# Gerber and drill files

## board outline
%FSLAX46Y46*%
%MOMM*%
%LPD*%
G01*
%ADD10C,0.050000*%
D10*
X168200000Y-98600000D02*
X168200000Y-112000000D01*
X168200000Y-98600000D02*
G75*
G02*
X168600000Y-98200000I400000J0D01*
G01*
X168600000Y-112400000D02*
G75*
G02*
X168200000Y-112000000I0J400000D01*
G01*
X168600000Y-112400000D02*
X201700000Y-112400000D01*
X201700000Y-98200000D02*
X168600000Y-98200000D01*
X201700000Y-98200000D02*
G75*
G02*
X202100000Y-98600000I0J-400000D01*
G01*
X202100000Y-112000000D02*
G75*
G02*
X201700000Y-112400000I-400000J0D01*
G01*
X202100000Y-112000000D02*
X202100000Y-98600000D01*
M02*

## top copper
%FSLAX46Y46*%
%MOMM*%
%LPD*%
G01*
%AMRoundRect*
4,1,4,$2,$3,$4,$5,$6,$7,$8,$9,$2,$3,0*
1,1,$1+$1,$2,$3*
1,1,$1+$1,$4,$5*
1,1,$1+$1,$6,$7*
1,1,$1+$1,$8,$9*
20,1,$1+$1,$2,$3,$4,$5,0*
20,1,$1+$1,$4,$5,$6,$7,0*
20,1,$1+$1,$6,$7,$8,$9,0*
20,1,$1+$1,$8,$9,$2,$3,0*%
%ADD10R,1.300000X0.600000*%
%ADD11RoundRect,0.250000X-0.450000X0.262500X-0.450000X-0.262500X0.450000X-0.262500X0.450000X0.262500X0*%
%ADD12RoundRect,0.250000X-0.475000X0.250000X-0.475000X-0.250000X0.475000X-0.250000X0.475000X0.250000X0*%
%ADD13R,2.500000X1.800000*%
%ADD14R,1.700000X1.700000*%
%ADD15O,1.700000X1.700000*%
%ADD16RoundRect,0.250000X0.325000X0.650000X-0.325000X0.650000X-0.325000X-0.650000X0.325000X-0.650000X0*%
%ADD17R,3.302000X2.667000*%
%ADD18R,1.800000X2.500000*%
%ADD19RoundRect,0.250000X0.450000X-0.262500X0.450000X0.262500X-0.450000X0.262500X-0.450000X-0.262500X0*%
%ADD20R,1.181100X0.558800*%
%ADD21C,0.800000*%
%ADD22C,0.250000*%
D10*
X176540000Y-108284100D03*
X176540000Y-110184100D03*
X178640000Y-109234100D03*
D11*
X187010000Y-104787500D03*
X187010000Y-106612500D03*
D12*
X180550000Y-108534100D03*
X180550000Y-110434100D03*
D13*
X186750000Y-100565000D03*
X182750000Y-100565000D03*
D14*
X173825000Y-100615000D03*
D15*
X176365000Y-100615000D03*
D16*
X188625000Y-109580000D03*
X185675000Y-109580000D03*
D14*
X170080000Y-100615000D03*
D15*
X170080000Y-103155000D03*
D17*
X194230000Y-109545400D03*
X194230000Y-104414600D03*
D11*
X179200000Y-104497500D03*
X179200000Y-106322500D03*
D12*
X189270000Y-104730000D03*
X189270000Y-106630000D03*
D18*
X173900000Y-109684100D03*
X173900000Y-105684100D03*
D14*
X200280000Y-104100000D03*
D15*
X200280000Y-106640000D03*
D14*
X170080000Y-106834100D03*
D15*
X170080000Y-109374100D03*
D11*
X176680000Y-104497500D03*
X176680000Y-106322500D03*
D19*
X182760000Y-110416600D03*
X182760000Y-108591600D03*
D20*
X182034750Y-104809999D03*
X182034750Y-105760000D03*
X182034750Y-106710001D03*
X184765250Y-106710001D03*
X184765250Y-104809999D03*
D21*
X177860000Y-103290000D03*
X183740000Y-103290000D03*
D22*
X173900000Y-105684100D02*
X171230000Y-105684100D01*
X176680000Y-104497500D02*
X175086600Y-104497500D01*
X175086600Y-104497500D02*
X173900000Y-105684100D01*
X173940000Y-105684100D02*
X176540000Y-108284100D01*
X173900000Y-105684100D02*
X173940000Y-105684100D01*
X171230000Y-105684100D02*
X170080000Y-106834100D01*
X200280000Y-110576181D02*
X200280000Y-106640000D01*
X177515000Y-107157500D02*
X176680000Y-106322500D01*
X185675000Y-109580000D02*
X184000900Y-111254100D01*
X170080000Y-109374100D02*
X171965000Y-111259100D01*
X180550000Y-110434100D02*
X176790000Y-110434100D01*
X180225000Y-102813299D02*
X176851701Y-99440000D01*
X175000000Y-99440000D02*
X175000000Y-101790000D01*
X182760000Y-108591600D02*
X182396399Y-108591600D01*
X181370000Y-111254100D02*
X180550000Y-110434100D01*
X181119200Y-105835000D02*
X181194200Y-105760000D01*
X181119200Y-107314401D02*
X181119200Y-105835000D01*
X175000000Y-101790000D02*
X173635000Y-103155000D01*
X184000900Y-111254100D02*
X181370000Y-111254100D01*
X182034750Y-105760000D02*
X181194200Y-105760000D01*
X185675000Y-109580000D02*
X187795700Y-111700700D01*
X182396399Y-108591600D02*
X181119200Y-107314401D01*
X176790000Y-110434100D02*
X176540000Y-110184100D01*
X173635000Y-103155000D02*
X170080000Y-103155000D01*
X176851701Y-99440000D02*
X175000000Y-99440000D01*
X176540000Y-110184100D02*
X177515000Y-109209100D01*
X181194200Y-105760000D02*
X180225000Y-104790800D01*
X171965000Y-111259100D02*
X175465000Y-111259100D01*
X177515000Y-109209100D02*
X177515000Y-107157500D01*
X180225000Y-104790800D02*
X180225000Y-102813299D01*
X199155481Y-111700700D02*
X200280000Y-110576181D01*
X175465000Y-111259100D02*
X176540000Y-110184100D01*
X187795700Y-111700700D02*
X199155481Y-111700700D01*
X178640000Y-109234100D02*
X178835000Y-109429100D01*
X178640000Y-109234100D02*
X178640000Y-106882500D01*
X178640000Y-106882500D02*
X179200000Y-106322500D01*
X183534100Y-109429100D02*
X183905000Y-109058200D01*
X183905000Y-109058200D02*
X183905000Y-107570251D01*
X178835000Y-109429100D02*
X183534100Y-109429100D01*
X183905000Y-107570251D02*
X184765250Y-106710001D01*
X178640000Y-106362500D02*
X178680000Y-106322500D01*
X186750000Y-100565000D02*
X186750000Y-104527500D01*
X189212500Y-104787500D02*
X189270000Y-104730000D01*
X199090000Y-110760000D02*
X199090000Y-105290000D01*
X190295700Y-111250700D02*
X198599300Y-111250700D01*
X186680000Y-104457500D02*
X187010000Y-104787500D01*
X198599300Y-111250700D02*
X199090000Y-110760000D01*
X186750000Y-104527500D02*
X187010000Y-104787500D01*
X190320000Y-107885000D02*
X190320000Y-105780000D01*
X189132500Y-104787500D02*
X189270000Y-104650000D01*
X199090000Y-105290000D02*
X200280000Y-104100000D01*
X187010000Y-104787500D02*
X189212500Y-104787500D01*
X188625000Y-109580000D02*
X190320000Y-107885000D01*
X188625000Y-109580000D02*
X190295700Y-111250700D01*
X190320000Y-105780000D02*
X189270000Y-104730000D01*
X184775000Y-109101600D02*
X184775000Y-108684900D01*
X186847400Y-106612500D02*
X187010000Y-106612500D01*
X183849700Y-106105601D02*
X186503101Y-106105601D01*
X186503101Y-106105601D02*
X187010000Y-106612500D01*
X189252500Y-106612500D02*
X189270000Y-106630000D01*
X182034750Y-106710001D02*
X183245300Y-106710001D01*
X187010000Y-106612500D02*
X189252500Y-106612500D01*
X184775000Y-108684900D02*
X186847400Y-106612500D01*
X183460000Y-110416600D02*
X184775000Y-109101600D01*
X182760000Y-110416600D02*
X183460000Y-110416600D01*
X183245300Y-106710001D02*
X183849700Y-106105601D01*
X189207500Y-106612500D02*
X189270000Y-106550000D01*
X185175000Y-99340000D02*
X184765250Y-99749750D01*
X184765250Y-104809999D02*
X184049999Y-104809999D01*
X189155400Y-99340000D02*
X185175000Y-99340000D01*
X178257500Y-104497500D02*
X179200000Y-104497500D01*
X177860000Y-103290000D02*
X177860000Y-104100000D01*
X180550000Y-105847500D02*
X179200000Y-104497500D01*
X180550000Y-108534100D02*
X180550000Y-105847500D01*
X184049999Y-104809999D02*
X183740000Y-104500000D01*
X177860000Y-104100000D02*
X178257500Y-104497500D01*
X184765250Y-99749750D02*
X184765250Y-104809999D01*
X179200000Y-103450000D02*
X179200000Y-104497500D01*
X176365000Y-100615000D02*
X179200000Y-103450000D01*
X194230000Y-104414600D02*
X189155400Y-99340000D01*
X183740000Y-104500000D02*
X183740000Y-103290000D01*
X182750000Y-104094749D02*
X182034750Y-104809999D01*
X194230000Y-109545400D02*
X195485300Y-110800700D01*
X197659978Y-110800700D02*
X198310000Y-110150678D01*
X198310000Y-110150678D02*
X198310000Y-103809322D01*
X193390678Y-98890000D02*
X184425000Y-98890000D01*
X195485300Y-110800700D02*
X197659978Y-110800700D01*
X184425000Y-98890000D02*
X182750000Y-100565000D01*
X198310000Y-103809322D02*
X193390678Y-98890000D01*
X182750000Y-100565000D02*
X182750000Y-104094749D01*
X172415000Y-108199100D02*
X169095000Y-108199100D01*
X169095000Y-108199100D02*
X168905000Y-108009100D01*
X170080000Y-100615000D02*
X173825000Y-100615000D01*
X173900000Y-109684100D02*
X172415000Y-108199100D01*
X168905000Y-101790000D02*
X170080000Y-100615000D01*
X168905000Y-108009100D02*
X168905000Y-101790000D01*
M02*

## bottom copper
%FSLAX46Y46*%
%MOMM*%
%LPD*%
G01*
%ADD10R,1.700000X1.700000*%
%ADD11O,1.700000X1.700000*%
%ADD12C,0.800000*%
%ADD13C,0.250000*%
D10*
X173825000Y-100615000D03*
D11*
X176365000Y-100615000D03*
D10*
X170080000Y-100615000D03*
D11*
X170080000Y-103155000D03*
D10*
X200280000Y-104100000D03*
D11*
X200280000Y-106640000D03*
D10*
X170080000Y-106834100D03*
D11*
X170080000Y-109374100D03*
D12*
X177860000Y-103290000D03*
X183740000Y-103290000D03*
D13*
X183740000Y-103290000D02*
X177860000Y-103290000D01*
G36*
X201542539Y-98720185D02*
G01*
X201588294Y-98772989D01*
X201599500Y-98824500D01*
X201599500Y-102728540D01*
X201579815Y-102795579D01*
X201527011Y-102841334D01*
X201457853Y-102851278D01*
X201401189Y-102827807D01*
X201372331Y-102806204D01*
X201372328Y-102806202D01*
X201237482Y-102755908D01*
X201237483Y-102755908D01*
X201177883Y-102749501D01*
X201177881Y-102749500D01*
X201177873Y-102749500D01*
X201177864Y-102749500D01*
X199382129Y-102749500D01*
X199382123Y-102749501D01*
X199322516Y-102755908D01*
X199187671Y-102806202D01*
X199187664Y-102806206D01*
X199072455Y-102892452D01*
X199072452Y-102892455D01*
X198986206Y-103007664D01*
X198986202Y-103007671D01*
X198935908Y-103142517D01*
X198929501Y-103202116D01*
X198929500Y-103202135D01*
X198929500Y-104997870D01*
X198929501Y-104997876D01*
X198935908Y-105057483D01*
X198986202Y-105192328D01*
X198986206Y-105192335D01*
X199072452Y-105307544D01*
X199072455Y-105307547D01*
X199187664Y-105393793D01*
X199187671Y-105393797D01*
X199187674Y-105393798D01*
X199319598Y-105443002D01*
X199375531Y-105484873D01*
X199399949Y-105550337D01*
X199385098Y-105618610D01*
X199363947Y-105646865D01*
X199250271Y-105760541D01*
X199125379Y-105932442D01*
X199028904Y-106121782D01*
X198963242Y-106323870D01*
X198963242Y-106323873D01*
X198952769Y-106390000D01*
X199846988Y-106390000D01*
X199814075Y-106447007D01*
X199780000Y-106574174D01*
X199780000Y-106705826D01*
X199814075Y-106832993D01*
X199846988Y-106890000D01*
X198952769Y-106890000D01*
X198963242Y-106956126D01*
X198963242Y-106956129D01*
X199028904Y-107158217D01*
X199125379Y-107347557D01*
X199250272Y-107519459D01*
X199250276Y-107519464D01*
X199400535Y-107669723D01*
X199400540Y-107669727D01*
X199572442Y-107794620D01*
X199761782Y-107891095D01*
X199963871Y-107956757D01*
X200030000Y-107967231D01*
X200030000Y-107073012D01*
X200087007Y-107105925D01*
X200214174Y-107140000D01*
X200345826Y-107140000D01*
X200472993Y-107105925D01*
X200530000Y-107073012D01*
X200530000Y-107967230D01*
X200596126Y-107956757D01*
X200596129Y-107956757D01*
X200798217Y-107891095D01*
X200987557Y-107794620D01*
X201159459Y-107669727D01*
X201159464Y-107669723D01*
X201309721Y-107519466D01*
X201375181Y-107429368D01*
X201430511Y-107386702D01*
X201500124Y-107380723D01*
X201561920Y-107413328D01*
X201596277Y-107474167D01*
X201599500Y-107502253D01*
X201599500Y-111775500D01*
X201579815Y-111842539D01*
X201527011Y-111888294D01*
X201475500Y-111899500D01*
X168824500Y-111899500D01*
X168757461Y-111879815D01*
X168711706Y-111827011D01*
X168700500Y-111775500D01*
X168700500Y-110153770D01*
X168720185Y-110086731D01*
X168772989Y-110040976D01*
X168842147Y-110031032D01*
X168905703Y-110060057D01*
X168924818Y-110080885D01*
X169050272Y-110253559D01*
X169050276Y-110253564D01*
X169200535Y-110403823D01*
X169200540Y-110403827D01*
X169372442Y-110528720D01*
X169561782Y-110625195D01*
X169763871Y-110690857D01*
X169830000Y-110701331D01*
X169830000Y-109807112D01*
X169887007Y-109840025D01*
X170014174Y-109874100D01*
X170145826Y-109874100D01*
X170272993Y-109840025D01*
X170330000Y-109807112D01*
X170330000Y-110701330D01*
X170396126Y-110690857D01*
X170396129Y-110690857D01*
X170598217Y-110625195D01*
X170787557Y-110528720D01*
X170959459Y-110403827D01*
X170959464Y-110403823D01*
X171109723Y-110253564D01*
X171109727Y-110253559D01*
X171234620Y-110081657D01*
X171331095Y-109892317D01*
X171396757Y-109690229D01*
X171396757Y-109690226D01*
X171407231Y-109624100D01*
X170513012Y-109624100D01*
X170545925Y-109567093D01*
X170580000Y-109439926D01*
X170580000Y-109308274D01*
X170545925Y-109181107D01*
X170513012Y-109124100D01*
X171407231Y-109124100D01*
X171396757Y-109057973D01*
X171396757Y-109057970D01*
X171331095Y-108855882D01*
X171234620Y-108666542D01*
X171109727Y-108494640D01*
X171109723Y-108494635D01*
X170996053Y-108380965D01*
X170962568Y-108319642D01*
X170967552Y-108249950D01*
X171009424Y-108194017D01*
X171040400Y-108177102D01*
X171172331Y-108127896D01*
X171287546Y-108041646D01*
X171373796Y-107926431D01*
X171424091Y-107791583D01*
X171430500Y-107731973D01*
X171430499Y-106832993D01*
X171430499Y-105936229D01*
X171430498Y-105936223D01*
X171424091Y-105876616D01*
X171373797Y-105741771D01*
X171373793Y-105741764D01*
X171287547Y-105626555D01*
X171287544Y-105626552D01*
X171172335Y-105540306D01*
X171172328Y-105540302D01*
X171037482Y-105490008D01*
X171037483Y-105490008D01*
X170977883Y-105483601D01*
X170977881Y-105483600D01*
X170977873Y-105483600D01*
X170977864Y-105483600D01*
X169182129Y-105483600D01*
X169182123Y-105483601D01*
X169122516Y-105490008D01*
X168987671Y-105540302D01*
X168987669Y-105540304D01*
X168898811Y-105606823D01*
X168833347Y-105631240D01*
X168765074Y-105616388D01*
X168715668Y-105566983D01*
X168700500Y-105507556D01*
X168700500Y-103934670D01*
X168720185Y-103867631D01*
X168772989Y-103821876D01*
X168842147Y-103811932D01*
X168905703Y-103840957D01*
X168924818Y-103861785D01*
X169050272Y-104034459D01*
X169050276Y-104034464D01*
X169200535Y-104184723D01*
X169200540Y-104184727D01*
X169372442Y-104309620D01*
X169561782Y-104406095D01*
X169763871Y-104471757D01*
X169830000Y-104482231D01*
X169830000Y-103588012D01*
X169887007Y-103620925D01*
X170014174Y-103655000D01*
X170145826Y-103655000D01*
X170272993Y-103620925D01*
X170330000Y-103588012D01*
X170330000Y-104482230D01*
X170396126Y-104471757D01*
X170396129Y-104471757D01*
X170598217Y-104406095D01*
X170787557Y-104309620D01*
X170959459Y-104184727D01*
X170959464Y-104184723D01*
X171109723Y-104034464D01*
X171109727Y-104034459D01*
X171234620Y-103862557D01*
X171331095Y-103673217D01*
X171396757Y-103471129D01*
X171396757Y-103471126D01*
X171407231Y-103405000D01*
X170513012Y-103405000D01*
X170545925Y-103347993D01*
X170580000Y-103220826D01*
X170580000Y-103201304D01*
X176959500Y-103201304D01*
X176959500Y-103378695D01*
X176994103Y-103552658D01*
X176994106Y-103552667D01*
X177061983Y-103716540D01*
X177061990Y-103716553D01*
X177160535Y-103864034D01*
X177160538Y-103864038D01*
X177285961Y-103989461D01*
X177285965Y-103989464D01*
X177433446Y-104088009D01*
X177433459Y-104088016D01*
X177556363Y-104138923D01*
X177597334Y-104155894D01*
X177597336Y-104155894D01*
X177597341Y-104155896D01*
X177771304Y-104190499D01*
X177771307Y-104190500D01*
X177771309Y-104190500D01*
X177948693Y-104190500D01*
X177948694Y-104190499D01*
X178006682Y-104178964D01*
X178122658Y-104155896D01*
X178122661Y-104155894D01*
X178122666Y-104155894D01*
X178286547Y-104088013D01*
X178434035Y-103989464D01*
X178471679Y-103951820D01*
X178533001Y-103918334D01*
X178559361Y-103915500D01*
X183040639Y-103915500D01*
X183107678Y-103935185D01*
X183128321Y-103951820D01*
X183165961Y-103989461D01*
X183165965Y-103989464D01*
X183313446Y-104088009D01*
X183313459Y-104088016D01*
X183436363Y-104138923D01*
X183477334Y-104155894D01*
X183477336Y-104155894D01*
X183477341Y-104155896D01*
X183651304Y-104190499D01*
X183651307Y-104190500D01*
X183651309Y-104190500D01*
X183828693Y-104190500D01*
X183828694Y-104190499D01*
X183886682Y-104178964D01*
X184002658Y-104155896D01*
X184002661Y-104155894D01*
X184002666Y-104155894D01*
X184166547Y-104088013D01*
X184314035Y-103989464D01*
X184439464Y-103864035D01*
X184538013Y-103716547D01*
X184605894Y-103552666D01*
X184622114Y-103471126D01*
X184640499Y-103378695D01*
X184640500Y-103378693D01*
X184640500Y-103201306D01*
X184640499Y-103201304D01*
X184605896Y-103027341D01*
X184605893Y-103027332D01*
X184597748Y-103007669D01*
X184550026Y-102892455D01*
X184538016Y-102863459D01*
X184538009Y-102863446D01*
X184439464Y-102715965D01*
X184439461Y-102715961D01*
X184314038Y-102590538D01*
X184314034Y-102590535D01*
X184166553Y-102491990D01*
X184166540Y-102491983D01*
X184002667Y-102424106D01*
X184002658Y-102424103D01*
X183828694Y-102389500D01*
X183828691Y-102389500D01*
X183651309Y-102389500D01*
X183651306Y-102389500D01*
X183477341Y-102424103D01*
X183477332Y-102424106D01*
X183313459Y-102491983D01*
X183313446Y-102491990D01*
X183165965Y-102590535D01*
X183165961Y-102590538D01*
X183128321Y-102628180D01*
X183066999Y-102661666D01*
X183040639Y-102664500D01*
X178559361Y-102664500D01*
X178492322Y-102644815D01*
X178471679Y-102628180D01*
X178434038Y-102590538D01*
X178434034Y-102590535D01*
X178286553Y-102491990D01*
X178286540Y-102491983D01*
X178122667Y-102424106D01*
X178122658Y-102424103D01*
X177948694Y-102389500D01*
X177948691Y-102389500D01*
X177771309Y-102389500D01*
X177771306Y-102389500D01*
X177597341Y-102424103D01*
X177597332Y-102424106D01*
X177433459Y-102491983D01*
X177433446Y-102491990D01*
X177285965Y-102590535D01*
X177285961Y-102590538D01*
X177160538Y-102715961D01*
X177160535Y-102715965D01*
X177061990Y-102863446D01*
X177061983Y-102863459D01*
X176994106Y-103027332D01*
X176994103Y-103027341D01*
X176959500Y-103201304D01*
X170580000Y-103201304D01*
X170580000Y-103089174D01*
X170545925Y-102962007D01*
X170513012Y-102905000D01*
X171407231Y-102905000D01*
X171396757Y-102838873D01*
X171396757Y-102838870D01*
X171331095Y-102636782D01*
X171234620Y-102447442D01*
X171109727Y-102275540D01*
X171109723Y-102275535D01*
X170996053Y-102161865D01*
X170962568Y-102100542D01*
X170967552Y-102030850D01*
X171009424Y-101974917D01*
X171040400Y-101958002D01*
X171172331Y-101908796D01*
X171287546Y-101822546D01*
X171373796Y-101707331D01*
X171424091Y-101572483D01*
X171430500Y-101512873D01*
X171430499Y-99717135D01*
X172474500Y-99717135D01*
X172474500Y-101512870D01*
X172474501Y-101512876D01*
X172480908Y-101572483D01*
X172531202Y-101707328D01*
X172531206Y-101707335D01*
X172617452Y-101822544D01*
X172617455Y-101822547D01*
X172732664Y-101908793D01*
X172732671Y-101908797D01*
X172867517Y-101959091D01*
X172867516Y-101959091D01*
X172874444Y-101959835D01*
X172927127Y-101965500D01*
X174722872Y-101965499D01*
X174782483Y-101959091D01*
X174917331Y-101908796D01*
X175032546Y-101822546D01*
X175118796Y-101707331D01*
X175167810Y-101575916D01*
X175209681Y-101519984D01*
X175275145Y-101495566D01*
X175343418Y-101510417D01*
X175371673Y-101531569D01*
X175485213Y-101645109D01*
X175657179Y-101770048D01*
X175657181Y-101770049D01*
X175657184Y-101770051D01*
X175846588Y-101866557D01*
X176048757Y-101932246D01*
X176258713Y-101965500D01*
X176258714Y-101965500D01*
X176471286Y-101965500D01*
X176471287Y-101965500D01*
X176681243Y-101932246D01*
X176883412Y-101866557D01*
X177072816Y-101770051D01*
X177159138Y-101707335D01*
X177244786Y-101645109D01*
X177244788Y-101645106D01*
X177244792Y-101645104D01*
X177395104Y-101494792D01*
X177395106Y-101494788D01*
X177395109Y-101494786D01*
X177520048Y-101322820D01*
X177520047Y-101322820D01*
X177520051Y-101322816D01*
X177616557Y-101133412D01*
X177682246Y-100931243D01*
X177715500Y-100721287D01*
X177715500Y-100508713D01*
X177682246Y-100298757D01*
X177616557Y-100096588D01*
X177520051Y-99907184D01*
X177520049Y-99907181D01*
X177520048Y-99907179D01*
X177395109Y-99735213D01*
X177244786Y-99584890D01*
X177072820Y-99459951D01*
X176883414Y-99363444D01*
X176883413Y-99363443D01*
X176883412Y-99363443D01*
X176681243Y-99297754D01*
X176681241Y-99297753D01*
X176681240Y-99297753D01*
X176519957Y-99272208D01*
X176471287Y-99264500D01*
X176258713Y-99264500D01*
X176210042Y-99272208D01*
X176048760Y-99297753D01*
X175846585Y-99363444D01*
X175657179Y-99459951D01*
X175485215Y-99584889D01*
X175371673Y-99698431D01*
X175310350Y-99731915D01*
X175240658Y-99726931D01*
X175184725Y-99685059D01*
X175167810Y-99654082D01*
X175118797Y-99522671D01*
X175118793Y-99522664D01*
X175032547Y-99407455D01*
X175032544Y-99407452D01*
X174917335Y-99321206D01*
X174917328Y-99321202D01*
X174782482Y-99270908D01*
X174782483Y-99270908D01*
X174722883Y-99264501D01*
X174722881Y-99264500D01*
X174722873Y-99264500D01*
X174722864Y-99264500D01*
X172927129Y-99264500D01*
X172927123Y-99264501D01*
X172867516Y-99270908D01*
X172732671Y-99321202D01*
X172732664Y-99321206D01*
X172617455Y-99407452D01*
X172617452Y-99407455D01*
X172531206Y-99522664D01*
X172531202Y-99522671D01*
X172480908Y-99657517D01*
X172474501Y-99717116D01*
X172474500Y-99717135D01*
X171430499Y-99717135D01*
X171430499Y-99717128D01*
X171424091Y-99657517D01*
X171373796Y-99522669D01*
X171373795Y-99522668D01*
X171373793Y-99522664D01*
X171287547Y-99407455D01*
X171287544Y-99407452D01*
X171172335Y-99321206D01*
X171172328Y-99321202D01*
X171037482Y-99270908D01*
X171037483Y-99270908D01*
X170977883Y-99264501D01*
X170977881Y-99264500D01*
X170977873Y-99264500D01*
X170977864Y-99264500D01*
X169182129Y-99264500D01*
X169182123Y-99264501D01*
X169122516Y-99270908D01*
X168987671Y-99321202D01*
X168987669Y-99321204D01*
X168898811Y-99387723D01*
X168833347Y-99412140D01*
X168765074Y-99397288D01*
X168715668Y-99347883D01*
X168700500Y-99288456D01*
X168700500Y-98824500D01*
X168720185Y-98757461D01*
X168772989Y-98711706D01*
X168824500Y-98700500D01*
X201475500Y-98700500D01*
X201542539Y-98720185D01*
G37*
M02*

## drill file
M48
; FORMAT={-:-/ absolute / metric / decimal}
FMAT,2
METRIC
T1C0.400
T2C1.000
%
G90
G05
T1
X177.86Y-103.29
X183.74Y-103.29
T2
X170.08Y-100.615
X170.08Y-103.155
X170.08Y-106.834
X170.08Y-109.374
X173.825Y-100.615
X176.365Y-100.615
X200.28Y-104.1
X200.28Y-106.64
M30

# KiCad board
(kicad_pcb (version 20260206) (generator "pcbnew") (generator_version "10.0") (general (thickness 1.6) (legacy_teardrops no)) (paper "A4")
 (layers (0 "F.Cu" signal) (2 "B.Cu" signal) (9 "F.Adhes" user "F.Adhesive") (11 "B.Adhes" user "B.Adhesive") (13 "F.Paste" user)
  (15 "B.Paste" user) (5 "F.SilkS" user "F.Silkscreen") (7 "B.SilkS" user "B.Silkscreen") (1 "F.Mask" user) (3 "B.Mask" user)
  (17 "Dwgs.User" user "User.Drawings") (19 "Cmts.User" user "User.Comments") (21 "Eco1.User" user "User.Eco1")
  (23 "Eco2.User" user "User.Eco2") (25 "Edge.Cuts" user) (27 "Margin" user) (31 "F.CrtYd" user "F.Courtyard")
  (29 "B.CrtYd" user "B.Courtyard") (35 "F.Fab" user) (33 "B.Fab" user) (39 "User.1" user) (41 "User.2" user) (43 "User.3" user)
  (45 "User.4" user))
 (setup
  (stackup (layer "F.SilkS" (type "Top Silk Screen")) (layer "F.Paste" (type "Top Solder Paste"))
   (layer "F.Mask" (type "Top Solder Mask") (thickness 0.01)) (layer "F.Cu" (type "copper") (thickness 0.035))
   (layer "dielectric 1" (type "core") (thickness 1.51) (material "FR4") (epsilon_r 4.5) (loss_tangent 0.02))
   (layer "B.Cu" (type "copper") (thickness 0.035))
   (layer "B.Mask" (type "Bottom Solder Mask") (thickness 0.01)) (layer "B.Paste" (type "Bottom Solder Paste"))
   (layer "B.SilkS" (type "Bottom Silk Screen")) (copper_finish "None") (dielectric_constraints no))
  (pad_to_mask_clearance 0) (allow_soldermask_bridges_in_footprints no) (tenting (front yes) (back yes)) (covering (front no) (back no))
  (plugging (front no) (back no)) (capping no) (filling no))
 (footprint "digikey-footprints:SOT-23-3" (layer "F.Cu") (at 177.59 109.2341)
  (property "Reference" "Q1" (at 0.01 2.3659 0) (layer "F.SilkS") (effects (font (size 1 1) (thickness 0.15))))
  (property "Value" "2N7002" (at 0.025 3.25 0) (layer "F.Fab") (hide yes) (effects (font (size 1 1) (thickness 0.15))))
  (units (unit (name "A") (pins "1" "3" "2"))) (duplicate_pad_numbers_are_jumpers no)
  (pad "1" smd rect (at -1.05 -0.95) (size 1.3 0.6) (layers "F.Cu" "F.Mask" "F.Paste") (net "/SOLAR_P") (solder_mask_margin 0.07))
  (pad "2" smd rect (at -1.05 0.95) (size 1.3 0.6) (layers "F.Cu" "F.Mask" "F.Paste") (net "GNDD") (solder_mask_margin 0.07))
  (pad "3" smd rect (at 1.05 0) (size 1.3 0.6) (layers "F.Cu" "F.Mask" "F.Paste") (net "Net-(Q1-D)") (solder_mask_margin 0.07)))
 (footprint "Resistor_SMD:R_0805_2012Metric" (layer "F.Cu") (at 187.01 105.7 -90)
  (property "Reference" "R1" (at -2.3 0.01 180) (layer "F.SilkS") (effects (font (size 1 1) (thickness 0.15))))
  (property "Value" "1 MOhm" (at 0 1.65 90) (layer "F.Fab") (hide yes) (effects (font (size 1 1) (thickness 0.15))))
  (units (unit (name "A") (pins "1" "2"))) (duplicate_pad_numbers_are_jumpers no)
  (pad "1" smd roundrect (at -0.9125 0 270) (size 1.025 1.4) (layers "F.Cu" "F.Mask" "F.Paste") (roundrect_rratio 0.243902) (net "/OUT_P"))
  (pad "2" smd roundrect (at 0.9125 0 270) (size 1.025 1.4) (layers "F.Cu" "F.Mask" "F.Paste") (roundrect_rratio 0.243902)
   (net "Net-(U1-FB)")))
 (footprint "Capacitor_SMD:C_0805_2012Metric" (layer "F.Cu") (at 180.55 109.4841 -90)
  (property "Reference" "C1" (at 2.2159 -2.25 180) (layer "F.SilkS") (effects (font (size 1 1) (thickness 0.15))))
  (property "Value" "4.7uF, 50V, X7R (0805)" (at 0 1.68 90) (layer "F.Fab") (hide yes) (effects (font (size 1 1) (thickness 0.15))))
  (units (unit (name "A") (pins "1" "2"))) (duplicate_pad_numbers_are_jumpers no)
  (pad "1" smd roundrect (at -0.95 0 270) (size 1 1.45) (layers "F.Cu" "F.Mask" "F.Paste") (roundrect_rratio 0.25) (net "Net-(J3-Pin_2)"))
  (pad "2" smd roundrect (at 0.95 0 270) (size 1 1.45) (layers "F.Cu" "F.Mask" "F.Paste") (roundrect_rratio 0.25) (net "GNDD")))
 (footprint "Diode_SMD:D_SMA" (layer "F.Cu") (at 184.75 100.565 180)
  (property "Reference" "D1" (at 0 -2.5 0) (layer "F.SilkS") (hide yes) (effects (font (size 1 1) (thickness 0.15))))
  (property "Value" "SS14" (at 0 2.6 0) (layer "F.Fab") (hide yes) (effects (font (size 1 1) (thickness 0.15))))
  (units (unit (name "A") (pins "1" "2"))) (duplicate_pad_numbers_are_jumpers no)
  (pad "1" smd rect (at -2 0 180) (size 2.5 1.8) (layers "F.Cu" "F.Mask" "F.Paste") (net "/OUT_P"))
  (pad "2" smd rect (at 2 0 180) (size 2.5 1.8) (layers "F.Cu" "F.Mask" "F.Paste") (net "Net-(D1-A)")))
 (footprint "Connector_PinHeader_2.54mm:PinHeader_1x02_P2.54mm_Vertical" (layer "F.Cu") (at 173.825 100.615 90)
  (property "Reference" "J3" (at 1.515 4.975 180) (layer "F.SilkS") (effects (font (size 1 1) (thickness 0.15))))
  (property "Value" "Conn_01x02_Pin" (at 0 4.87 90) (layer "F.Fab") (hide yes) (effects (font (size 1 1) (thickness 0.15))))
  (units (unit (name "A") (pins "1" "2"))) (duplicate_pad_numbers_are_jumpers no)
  (pad "1" thru_hole rect (at 0 0 90) (size 1.7 1.7) (drill 1) (layers "*.Cu" "*.Mask") (remove_unused_layers no) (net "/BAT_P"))
  (pad "2" thru_hole oval (at 0 2.54 90) (size 1.7 1.7) (drill 1) (layers "*.Cu" "*.Mask") (remove_unused_layers no) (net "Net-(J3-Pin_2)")))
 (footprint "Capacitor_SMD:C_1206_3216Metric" (layer "F.Cu") (at 187.15 109.58 180)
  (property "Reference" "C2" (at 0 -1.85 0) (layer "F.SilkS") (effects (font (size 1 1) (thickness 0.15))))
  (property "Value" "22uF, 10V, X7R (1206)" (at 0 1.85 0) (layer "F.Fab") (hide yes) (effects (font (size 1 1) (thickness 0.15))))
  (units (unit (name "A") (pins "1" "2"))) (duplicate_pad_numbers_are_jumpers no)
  (pad "1" smd roundrect (at -1.475 0 180) (size 1.15 1.8) (layers "F.Cu" "F.Mask" "F.Paste") (roundrect_rratio 0.217391) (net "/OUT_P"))
  (pad "2" smd roundrect (at 1.475 0 180) (size 1.15 1.8) (layers "F.Cu" "F.Mask" "F.Paste") (roundrect_rratio 0.217391) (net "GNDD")))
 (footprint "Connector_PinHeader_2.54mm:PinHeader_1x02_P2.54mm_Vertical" (layer "F.Cu") (at 170.08 100.615)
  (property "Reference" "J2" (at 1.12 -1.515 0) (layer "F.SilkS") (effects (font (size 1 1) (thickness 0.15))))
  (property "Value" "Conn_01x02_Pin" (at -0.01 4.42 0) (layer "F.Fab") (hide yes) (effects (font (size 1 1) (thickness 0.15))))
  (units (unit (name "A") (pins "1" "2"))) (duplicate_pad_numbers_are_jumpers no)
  (pad "1" thru_hole rect (at 0 0) (size 1.7 1.7) (drill 1) (layers "*.Cu" "*.Mask") (remove_unused_layers no) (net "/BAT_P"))
  (pad "2" thru_hole oval (at 0 2.54) (size 1.7 1.7) (drill 1) (layers "*.Cu" "*.Mask") (remove_unused_layers no) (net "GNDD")))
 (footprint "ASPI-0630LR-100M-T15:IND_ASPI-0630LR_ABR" (layer "F.Cu") (at 194.23 106.98 90)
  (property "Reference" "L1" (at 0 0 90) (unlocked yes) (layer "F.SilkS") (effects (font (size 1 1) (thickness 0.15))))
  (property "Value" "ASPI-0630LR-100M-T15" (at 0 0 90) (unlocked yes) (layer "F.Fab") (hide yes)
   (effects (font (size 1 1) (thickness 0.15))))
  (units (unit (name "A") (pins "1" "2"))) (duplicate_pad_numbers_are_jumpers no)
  (pad "1" smd rect (at -2.5654 0 180) (size 3.302 2.667) (layers "F.Cu" "F.Mask" "F.Paste") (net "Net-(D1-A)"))
  (pad "2" smd rect (at 2.5654 0 180) (size 3.302 2.667) (layers "F.Cu" "F.Mask" "F.Paste") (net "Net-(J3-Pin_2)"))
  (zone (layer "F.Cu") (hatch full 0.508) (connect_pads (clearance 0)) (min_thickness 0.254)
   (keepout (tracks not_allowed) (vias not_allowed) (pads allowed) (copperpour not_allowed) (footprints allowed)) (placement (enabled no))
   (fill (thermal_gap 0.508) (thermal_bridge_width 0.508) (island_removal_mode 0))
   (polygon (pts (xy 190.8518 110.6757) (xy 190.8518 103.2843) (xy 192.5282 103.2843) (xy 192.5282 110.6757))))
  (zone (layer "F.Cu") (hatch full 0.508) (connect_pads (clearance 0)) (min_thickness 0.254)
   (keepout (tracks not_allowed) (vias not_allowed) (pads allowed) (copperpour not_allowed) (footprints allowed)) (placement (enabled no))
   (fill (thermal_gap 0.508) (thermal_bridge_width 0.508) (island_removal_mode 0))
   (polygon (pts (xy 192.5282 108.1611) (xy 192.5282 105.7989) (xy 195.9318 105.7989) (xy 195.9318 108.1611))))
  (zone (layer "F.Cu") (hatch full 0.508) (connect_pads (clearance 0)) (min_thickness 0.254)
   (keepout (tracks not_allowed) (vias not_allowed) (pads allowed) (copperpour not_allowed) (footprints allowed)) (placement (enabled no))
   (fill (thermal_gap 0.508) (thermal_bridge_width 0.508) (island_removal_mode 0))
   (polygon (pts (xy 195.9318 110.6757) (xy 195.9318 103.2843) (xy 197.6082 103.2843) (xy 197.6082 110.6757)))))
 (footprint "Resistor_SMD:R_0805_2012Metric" (layer "F.Cu") (at 179.2 105.41 -90)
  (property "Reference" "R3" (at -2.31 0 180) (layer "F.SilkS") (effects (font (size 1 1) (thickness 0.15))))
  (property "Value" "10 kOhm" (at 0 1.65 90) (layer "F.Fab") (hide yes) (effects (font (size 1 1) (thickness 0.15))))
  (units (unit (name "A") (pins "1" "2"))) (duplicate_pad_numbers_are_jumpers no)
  (pad "1" smd roundrect (at -0.9125 0 270) (size 1.025 1.4) (layers "F.Cu" "F.Mask" "F.Paste") (roundrect_rratio 0.243902)
   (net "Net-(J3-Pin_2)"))
  (pad "2" smd roundrect (at 0.9125 0 270) (size 1.025 1.4) (layers "F.Cu" "F.Mask" "F.Paste") (roundrect_rratio 0.243902)
   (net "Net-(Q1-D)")))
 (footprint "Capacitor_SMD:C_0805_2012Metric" (layer "F.Cu") (at 189.27 105.68 -90)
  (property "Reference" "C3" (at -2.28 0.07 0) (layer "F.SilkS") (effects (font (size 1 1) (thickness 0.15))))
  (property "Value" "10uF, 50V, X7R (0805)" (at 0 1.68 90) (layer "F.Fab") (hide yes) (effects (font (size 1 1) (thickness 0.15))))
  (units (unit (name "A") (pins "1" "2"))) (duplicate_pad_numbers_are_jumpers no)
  (pad "1" smd roundrect (at -0.95 0 270) (size 1 1.45) (layers "F.Cu" "F.Mask" "F.Paste") (roundrect_rratio 0.25) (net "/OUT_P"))
  (pad "2" smd roundrect (at 0.95 0 270) (size 1 1.45) (layers "F.Cu" "F.Mask" "F.Paste") (roundrect_rratio 0.25) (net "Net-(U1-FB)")))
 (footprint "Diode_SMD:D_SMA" (layer "F.Cu") (at 173.9 107.6841 90)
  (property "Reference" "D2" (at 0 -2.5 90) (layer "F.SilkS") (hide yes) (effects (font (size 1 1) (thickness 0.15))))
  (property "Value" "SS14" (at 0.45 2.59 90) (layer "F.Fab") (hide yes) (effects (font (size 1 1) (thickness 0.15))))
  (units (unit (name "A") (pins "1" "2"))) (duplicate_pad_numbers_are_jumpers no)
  (pad "1" smd rect (at -2 0 90) (size 2.5 1.8) (layers "F.Cu" "F.Mask" "F.Paste") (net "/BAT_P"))
  (pad "2" smd rect (at 2 0 90) (size 2.5 1.8) (layers "F.Cu" "F.Mask" "F.Paste") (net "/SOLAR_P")))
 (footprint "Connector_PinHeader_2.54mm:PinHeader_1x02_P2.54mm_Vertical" (layer "F.Cu") (at 200.28 104.1)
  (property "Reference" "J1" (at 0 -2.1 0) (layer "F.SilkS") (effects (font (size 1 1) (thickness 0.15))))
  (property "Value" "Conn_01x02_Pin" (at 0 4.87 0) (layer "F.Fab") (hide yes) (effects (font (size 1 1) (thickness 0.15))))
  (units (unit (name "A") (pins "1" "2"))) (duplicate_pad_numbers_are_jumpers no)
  (pad "1" thru_hole rect (at 0 0) (size 1.7 1.7) (drill 1) (layers "*.Cu" "*.Mask") (remove_unused_layers no) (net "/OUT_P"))
  (pad "2" thru_hole oval (at 0 2.54) (size 1.7 1.7) (drill 1) (layers "*.Cu" "*.Mask") (remove_unused_layers no) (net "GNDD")))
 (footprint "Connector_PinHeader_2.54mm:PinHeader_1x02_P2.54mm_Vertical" (layer "F.Cu") (at 170.08 106.8341)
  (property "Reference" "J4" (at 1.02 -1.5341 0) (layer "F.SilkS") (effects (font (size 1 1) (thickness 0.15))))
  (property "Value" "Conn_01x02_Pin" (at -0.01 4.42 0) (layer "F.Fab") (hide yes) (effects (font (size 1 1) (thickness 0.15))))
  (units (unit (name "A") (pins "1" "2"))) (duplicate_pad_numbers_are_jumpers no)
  (pad "1" thru_hole rect (at 0 0) (size 1.7 1.7) (drill 1) (layers "*.Cu" "*.Mask") (remove_unused_layers no) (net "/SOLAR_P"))
  (pad "2" thru_hole oval (at 0 2.54) (size 1.7 1.7) (drill 1) (layers "*.Cu" "*.Mask") (remove_unused_layers no) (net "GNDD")))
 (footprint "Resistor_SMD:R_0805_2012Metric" (layer "F.Cu") (at 176.68 105.41 -90)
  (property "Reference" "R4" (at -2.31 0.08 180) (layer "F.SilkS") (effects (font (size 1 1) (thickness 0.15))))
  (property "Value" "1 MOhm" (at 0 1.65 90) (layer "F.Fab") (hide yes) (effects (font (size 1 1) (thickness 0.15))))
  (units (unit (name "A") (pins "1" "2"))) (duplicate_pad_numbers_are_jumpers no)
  (pad "1" smd roundrect (at -0.9125 0 270) (size 1.025 1.4) (layers "F.Cu" "F.Mask" "F.Paste") (roundrect_rratio 0.243902) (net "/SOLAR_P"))
  (pad "2" smd roundrect (at 0.9125 0 270) (size 1.025 1.4) (layers "F.Cu" "F.Mask" "F.Paste") (roundrect_rratio 0.243902) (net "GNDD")))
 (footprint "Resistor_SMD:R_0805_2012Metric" (layer "F.Cu") (at 182.76 109.5041 90)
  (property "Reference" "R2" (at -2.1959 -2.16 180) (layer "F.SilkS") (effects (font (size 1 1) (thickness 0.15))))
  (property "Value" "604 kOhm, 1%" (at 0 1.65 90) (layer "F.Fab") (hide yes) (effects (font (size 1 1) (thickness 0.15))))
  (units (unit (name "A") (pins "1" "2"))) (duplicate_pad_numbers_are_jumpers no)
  (pad "1" smd roundrect (at -0.9125 0 90) (size 1.025 1.4) (layers "F.Cu" "F.Mask" "F.Paste") (roundrect_rratio 0.243902)
   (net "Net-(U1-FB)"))
  (pad "2" smd roundrect (at 0.9125 0 90) (size 1.025 1.4) (layers "F.Cu" "F.Mask" "F.Paste") (roundrect_rratio 0.243902) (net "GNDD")))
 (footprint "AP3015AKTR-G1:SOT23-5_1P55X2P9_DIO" (layer "F.Cu") (at 183.4 105.76)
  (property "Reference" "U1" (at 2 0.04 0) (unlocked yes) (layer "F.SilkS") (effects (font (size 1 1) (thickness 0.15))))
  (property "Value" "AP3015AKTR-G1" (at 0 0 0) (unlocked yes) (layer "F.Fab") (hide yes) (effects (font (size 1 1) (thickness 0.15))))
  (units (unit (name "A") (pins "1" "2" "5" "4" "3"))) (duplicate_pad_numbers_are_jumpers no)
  (pad "1" smd rect (at -1.36525 -0.950001) (size 1.1811 0.5588) (layers "F.Cu" "F.Mask" "F.Paste") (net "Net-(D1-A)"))
  (pad "2" smd rect (at -1.36525 0) (size 1.1811 0.5588) (layers "F.Cu" "F.Mask" "F.Paste") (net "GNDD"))
  (pad "3" smd rect (at -1.36525 0.950001) (size 1.1811 0.5588) (layers "F.Cu" "F.Mask" "F.Paste") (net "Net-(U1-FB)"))
  (pad "4" smd rect (at 1.36525 0.950001) (size 1.1811 0.5588) (layers "F.Cu" "F.Mask" "F.Paste") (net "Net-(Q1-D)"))
  (pad "5" smd rect (at 1.36525 -0.950001) (size 1.1811 0.5588) (layers "F.Cu" "F.Mask" "F.Paste") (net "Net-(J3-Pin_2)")))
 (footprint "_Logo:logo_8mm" (layer "B.Cu") (at 185 100.6 180)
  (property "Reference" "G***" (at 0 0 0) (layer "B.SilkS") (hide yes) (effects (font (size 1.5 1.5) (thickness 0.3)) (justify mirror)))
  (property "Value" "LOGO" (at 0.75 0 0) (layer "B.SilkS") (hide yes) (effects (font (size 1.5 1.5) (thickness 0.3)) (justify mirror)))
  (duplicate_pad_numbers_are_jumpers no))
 (gr_line (start 168.2 98.6) (end 168.2 112) (stroke (width 0.05) (type default)) (layer "Edge.Cuts"))
 (gr_arc (start 168.2 98.6) (mid 168.317157 98.317157) (end 168.6 98.2) (stroke (width 0.05) (type default)) (layer "Edge.Cuts"))
 (gr_arc (start 168.6 112.4) (mid 168.317157 112.282843) (end 168.2 112) (stroke (width 0.05) (type default)) (layer "Edge.Cuts"))
 (gr_line (start 168.6 112.4) (end 201.7 112.4) (stroke (width 0.05) (type default)) (layer "Edge.Cuts"))
 (gr_line (start 201.7 98.2) (end 168.6 98.2) (stroke (width 0.05) (type default)) (layer "Edge.Cuts"))
 (gr_arc (start 201.7 98.2) (mid 201.982843 98.317157) (end 202.1 98.6) (stroke (width 0.05) (type default)) (layer "Edge.Cuts"))
 (gr_arc (start 202.1 112) (mid 201.982843 112.282843) (end 201.7 112.4) (stroke (width 0.05) (type default)) (layer "Edge.Cuts"))
 (gr_line (start 202.1 112) (end 202.1 98.6) (stroke (width 0.05) (type default)) (layer "Edge.Cuts"))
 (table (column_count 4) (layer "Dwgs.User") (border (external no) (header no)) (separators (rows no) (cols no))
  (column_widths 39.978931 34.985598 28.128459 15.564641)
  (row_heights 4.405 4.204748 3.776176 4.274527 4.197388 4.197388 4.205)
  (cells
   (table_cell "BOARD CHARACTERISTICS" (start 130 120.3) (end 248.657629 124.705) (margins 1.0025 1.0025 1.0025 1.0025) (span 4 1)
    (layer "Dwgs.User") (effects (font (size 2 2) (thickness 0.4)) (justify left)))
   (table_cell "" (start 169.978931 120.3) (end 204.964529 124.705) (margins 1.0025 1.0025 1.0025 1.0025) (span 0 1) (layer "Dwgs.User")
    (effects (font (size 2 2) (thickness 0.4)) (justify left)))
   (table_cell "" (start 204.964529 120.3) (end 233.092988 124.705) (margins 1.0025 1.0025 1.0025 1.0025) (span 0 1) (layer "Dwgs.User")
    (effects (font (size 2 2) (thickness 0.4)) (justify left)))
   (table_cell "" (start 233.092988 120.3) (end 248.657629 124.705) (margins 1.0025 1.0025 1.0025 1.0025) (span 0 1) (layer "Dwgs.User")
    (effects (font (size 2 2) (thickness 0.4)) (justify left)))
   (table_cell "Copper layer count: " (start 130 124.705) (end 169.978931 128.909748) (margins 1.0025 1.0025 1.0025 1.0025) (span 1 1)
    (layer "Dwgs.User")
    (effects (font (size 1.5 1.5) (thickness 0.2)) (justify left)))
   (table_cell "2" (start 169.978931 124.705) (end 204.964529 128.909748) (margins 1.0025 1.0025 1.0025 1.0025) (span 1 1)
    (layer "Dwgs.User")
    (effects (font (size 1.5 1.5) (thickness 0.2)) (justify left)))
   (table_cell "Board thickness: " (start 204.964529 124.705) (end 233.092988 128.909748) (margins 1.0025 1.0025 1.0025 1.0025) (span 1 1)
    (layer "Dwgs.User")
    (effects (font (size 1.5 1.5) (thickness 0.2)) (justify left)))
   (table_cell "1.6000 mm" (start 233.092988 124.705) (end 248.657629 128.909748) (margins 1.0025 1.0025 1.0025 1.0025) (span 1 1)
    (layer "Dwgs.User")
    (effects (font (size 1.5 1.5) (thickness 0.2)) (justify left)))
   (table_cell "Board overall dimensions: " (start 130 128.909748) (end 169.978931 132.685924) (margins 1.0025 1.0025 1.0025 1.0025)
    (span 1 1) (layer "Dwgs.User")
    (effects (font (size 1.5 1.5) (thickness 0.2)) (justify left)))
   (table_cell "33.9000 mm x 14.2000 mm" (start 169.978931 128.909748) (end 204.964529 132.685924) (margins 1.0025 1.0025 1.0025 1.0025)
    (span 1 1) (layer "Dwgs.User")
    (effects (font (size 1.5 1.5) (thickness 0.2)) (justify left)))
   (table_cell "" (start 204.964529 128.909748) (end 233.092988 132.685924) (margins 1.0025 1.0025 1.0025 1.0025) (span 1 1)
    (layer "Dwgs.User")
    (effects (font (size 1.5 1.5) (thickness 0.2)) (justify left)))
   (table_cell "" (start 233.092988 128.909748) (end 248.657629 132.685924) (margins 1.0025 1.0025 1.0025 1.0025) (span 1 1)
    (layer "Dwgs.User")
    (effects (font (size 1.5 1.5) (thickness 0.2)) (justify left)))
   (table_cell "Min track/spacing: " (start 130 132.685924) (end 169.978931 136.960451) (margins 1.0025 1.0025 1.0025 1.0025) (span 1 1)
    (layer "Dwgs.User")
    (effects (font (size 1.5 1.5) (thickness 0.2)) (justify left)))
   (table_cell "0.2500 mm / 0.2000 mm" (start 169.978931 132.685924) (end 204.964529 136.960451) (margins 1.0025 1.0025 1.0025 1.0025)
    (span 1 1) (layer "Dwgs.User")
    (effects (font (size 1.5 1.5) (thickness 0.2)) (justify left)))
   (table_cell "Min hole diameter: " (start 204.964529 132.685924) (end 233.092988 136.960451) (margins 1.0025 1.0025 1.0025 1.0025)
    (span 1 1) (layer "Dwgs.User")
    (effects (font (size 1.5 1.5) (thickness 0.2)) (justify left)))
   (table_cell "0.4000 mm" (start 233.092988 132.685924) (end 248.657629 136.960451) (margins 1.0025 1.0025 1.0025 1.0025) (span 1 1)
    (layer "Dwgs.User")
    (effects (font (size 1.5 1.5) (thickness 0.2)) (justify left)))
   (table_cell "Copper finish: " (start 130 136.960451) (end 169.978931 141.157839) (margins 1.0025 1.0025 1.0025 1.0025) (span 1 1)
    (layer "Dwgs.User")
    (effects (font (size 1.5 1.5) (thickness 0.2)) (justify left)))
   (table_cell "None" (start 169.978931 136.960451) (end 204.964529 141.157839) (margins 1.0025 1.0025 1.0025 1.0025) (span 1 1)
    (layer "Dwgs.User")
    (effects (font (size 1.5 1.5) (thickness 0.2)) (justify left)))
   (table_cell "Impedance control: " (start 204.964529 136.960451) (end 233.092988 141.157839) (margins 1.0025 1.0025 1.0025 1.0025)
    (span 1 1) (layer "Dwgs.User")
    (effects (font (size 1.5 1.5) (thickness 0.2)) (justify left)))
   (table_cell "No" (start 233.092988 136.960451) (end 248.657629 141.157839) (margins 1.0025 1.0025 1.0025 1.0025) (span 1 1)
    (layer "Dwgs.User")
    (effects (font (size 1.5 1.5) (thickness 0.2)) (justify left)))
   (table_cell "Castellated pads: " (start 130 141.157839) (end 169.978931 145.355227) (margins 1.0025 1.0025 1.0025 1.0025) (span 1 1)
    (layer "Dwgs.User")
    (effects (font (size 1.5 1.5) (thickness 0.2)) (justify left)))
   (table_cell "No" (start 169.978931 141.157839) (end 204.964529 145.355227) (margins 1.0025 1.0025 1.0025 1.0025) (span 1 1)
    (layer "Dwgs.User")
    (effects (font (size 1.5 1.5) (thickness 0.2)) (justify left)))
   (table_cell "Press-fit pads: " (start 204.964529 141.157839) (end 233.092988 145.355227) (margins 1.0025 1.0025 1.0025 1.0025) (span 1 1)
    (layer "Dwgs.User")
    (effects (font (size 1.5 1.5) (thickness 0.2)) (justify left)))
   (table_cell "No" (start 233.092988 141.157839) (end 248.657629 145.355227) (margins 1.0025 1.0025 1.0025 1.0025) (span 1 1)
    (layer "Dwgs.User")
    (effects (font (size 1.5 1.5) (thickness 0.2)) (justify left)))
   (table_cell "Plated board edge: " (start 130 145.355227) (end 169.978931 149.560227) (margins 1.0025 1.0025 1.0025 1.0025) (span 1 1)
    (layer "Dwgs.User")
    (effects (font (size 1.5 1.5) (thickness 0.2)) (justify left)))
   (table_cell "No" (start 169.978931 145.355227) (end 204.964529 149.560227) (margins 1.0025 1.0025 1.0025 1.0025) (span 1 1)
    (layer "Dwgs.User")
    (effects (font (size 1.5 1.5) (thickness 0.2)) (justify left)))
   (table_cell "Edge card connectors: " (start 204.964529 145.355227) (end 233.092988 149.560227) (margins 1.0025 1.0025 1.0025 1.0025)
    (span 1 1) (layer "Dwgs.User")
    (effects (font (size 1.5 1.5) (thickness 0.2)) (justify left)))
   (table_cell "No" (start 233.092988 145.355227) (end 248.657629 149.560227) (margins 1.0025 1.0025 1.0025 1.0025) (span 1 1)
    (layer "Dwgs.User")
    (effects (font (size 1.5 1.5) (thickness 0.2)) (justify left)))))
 (segment (start 173.9 105.6841) (end 171.23 105.6841) (width 0.25) (layer "F.Cu") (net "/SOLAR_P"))
 (segment (start 176.68 104.4975) (end 175.0866 104.4975) (width 0.25) (layer "F.Cu") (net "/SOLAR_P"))
 (segment (start 175.0866 104.4975) (end 173.9 105.6841) (width 0.25) (layer "F.Cu") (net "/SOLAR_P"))
 (segment (start 173.94 105.6841) (end 176.54 108.2841) (width 0.25) (layer "F.Cu") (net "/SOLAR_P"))
 (segment (start 173.9 105.6841) (end 173.94 105.6841) (width 0.25) (layer "F.Cu") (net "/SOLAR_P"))
 (segment (start 171.23 105.6841) (end 170.08 106.8341) (width 0.25) (layer "F.Cu") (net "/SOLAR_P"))
 (segment (start 200.28 110.576181) (end 200.28 106.64) (width 0.25) (layer "F.Cu") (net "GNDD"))
 (segment (start 177.515 107.1575) (end 176.68 106.3225) (width 0.25) (layer "F.Cu") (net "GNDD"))
 (segment (start 185.675 109.58) (end 184.0009 111.2541) (width 0.25) (layer "F.Cu") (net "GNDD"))
 (segment (start 170.08 109.3741) (end 171.965 111.2591) (width 0.25) (layer "F.Cu") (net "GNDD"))
 (segment (start 180.55 110.4341) (end 176.79 110.4341) (width 0.25) (layer "F.Cu") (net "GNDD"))
 (segment (start 180.225 102.813299) (end 176.851701 99.44) (width 0.25) (layer "F.Cu") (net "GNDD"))
 (segment (start 175 99.44) (end 175 101.79) (width 0.25) (layer "F.Cu") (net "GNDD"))
 (segment (start 182.76 108.5916) (end 182.396399 108.5916) (width 0.25) (layer "F.Cu") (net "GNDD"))
 (segment (start 181.37 111.2541) (end 180.55 110.4341) (width 0.25) (layer "F.Cu") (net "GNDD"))
 (segment (start 181.1192 105.835) (end 181.1942 105.76) (width 0.25) (layer "F.Cu") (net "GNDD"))
 (segment (start 181.1192 107.314401) (end 181.1192 105.835) (width 0.25) (layer "F.Cu") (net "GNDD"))
 (segment (start 175 101.79) (end 173.635 103.155) (width 0.25) (layer "F.Cu") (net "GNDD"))
 (segment (start 184.0009 111.2541) (end 181.37 111.2541) (width 0.25) (layer "F.Cu") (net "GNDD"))
 (segment (start 182.03475 105.76) (end 181.1942 105.76) (width 0.25) (layer "F.Cu") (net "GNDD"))
 (segment (start 185.675 109.58) (end 187.7957 111.7007) (width 0.25) (layer "F.Cu") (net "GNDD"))
 (segment (start 182.396399 108.5916) (end 181.1192 107.314401) (width 0.25) (layer "F.Cu") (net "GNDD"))
 (segment (start 176.79 110.4341) (end 176.54 110.1841) (width 0.25) (layer "F.Cu") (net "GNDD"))
 (segment (start 173.635 103.155) (end 170.08 103.155) (width 0.25) (layer "F.Cu") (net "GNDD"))
 (segment (start 176.851701 99.44) (end 175 99.44) (width 0.25) (layer "F.Cu") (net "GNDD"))
 (segment (start 176.54 110.1841) (end 177.515 109.2091) (width 0.25) (layer "F.Cu") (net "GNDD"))
 (segment (start 181.1942 105.76) (end 180.225 104.7908) (width 0.25) (layer "F.Cu") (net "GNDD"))
 (segment (start 171.965 111.2591) (end 175.465 111.2591) (width 0.25) (layer "F.Cu") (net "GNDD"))
 (segment (start 177.515 109.2091) (end 177.515 107.1575) (width 0.25) (layer "F.Cu") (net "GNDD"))
 (segment (start 180.225 104.7908) (end 180.225 102.813299) (width 0.25) (layer "F.Cu") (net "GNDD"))
 (segment (start 199.155481 111.7007) (end 200.28 110.576181) (width 0.25) (layer "F.Cu") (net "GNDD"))
 (segment (start 175.465 111.2591) (end 176.54 110.1841) (width 0.25) (layer "F.Cu") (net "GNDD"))
 (segment (start 187.7957 111.7007) (end 199.155481 111.7007) (width 0.25) (layer "F.Cu") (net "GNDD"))
 (segment (start 178.64 109.2341) (end 178.835 109.4291) (width 0.25) (layer "F.Cu") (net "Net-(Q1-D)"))
 (segment (start 178.64 109.2341) (end 178.64 106.8825) (width 0.25) (layer "F.Cu") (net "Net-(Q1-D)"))
 (segment (start 178.64 106.8825) (end 179.2 106.3225) (width 0.25) (layer "F.Cu") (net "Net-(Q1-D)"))
 (segment (start 183.5341 109.4291) (end 183.905 109.0582) (width 0.25) (layer "F.Cu") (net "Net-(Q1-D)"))
 (segment (start 183.905 109.0582) (end 183.905 107.570251) (width 0.25) (layer "F.Cu") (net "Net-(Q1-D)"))
 (segment (start 178.835 109.4291) (end 183.5341 109.4291) (width 0.25) (layer "F.Cu") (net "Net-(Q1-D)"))
 (segment (start 183.905 107.570251) (end 184.76525 106.710001) (width 0.25) (layer "F.Cu") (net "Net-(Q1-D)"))
 (segment (start 178.64 106.3625) (end 178.68 106.3225) (width 0.25) (layer "F.Cu") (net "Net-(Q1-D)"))
 (segment (start 186.75 100.565) (end 186.75 104.5275) (width 0.25) (layer "F.Cu") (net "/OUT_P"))
 (segment (start 189.2125 104.7875) (end 189.27 104.73) (width 0.25) (layer "F.Cu") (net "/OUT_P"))
 (segment (start 199.09 110.76) (end 199.09 105.29) (width 0.25) (layer "F.Cu") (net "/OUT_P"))
 (segment (start 190.2957 111.2507) (end 198.5993 111.2507) (width 0.25) (layer "F.Cu") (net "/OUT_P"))
 (segment (start 186.68 104.4575) (end 187.01 104.7875) (width 0.25) (layer "F.Cu") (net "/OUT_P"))
 (segment (start 198.5993 111.2507) (end 199.09 110.76) (width 0.25) (layer "F.Cu") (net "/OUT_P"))
 (segment (start 186.75 104.5275) (end 187.01 104.7875) (width 0.25) (layer "F.Cu") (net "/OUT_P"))
 (segment (start 190.32 107.885) (end 190.32 105.78) (width 0.25) (layer "F.Cu") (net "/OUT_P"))
 (segment (start 189.1325 104.7875) (end 189.27 104.65) (width 0.25) (layer "F.Cu") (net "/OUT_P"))
 (segment (start 199.09 105.29) (end 200.28 104.1) (width 0.25) (layer "F.Cu") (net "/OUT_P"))
 (segment (start 187.01 104.7875) (end 189.2125 104.7875) (width 0.25) (layer "F.Cu") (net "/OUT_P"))
 (segment (start 188.625 109.58) (end 190.32 107.885) (width 0.25) (layer "F.Cu") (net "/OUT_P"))
 (segment (start 188.625 109.58) (end 190.2957 111.2507) (width 0.25) (layer "F.Cu") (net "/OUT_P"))
 (segment (start 190.32 105.78) (end 189.27 104.73) (width 0.25) (layer "F.Cu") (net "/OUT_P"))
 (segment (start 184.775 109.1016) (end 184.775 108.6849) (width 0.25) (layer "F.Cu") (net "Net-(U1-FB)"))
 (segment (start 186.8474 106.6125) (end 187.01 106.6125) (width 0.25) (layer "F.Cu") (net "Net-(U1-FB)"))
 (segment (start 183.8497 106.105601) (end 186.503101 106.105601) (width 0.25) (layer "F.Cu") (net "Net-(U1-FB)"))
 (segment (start 186.503101 106.105601) (end 187.01 106.6125) (width 0.25) (layer "F.Cu") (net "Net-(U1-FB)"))
 (segment (start 189.2525 106.6125) (end 189.27 106.63) (width 0.25) (layer "F.Cu") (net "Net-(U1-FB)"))
 (segment (start 182.03475 106.710001) (end 183.2453 106.710001) (width 0.25) (layer "F.Cu") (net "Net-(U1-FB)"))
 (segment (start 187.01 106.6125) (end 189.2525 106.6125) (width 0.25) (layer "F.Cu") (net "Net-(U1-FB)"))
 (segment (start 184.775 108.6849) (end 186.8474 106.6125) (width 0.25) (layer "F.Cu") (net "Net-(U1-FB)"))
 (segment (start 183.46 110.4166) (end 184.775 109.1016) (width 0.25) (layer "F.Cu") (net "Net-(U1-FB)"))
 (segment (start 182.76 110.4166) (end 183.46 110.4166) (width 0.25) (layer "F.Cu") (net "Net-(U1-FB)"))
 (segment (start 183.2453 106.710001) (end 183.8497 106.105601) (width 0.25) (layer "F.Cu") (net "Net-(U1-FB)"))
 (segment (start 189.2075 106.6125) (end 189.27 106.55) (width 0.25) (layer "F.Cu") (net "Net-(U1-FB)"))
 (segment (start 185.175 99.34) (end 184.76525 99.74975) (width 0.25) (layer "F.Cu") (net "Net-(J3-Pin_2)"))
 (segment (start 184.76525 104.809999) (end 184.049999 104.809999) (width 0.25) (layer "F.Cu") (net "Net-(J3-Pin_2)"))
 (segment (start 189.1554 99.34) (end 185.175 99.34) (width 0.25) (layer "F.Cu") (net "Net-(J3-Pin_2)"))
 (segment (start 178.2575 104.4975) (end 179.2 104.4975) (width 0.25) (layer "F.Cu") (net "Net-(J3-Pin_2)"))
 (segment (start 177.86 103.29) (end 177.86 104.1) (width 0.25) (layer "F.Cu") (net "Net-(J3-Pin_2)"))
 (segment (start 180.55 105.8475) (end 179.2 104.4975) (width 0.25) (layer "F.Cu") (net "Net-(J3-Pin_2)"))
 (segment (start 180.55 108.5341) (end 180.55 105.8475) (width 0.25) (layer "F.Cu") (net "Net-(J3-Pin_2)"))
 (segment (start 184.049999 104.809999) (end 183.74 104.5) (width 0.25) (layer "F.Cu") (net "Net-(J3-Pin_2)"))
 (segment (start 177.86 104.1) (end 178.2575 104.4975) (width 0.25) (layer "F.Cu") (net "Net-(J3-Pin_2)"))
 (segment (start 184.76525 99.74975) (end 184.76525 104.809999) (width 0.25) (layer "F.Cu") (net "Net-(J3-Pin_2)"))
 (segment (start 179.2 103.45) (end 179.2 104.4975) (width 0.25) (layer "F.Cu") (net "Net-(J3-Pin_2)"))
 (segment (start 176.365 100.615) (end 179.2 103.45) (width 0.25) (layer "F.Cu") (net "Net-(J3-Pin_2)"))
 (segment (start 194.23 104.4146) (end 189.1554 99.34) (width 0.25) (layer "F.Cu") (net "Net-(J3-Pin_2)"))
 (segment (start 183.74 104.5) (end 183.74 103.29) (width 0.25) (layer "F.Cu") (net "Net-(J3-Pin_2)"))
 (via (at 177.86 103.29) (size 0.8) (drill 0.4) (layers "F.Cu" "B.Cu") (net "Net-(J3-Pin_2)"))
 (via (at 183.74 103.29) (size 0.8) (drill 0.4) (layers "F.Cu" "B.Cu") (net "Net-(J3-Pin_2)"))
 (segment (start 183.74 103.29) (end 177.86 103.29) (width 0.25) (layer "B.Cu") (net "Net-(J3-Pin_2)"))
 (segment (start 182.75 104.094749) (end 182.03475 104.809999) (width 0.25) (layer "F.Cu") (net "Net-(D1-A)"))
 (segment (start 194.23 109.5454) (end 195.4853 110.8007) (width 0.25) (layer "F.Cu") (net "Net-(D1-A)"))
 (segment (start 197.659978 110.8007) (end 198.31 110.150678) (width 0.25) (layer "F.Cu") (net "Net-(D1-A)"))
 (segment (start 198.31 110.150678) (end 198.31 103.809322) (width 0.25) (layer "F.Cu") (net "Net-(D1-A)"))
 (segment (start 193.390678 98.89) (end 184.425 98.89) (width 0.25) (layer "F.Cu") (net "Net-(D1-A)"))
 (segment (start 195.4853 110.8007) (end 197.659978 110.8007) (width 0.25) (layer "F.Cu") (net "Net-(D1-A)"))
 (segment (start 184.425 98.89) (end 182.75 100.565) (width 0.25) (layer "F.Cu") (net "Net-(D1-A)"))
 (segment (start 198.31 103.809322) (end 193.390678 98.89) (width 0.25) (layer "F.Cu") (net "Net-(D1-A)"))
 (segment (start 182.75 100.565) (end 182.75 104.094749) (width 0.25) (layer "F.Cu") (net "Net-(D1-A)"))
 (segment (start 172.415 108.1991) (end 169.095 108.1991) (width 0.25) (layer "F.Cu") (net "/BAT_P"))
 (segment (start 169.095 108.1991) (end 168.905 108.0091) (width 0.25) (layer "F.Cu") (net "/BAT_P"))
 (segment (start 170.08 100.615) (end 173.825 100.615) (width 0.25) (layer "F.Cu") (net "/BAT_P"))
 (segment (start 173.9 109.6841) (end 172.415 108.1991) (width 0.25) (layer "F.Cu") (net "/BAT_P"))
 (segment (start 168.905 101.79) (end 170.08 100.615) (width 0.25) (layer "F.Cu") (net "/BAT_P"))
 (segment (start 168.905 108.0091) (end 168.905 101.79) (width 0.25) (layer "F.Cu") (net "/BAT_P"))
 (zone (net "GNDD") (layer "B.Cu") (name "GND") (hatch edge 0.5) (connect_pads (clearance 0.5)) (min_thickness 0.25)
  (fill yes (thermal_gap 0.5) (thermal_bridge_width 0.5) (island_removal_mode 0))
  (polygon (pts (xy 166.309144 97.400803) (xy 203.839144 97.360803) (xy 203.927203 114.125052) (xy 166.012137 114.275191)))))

